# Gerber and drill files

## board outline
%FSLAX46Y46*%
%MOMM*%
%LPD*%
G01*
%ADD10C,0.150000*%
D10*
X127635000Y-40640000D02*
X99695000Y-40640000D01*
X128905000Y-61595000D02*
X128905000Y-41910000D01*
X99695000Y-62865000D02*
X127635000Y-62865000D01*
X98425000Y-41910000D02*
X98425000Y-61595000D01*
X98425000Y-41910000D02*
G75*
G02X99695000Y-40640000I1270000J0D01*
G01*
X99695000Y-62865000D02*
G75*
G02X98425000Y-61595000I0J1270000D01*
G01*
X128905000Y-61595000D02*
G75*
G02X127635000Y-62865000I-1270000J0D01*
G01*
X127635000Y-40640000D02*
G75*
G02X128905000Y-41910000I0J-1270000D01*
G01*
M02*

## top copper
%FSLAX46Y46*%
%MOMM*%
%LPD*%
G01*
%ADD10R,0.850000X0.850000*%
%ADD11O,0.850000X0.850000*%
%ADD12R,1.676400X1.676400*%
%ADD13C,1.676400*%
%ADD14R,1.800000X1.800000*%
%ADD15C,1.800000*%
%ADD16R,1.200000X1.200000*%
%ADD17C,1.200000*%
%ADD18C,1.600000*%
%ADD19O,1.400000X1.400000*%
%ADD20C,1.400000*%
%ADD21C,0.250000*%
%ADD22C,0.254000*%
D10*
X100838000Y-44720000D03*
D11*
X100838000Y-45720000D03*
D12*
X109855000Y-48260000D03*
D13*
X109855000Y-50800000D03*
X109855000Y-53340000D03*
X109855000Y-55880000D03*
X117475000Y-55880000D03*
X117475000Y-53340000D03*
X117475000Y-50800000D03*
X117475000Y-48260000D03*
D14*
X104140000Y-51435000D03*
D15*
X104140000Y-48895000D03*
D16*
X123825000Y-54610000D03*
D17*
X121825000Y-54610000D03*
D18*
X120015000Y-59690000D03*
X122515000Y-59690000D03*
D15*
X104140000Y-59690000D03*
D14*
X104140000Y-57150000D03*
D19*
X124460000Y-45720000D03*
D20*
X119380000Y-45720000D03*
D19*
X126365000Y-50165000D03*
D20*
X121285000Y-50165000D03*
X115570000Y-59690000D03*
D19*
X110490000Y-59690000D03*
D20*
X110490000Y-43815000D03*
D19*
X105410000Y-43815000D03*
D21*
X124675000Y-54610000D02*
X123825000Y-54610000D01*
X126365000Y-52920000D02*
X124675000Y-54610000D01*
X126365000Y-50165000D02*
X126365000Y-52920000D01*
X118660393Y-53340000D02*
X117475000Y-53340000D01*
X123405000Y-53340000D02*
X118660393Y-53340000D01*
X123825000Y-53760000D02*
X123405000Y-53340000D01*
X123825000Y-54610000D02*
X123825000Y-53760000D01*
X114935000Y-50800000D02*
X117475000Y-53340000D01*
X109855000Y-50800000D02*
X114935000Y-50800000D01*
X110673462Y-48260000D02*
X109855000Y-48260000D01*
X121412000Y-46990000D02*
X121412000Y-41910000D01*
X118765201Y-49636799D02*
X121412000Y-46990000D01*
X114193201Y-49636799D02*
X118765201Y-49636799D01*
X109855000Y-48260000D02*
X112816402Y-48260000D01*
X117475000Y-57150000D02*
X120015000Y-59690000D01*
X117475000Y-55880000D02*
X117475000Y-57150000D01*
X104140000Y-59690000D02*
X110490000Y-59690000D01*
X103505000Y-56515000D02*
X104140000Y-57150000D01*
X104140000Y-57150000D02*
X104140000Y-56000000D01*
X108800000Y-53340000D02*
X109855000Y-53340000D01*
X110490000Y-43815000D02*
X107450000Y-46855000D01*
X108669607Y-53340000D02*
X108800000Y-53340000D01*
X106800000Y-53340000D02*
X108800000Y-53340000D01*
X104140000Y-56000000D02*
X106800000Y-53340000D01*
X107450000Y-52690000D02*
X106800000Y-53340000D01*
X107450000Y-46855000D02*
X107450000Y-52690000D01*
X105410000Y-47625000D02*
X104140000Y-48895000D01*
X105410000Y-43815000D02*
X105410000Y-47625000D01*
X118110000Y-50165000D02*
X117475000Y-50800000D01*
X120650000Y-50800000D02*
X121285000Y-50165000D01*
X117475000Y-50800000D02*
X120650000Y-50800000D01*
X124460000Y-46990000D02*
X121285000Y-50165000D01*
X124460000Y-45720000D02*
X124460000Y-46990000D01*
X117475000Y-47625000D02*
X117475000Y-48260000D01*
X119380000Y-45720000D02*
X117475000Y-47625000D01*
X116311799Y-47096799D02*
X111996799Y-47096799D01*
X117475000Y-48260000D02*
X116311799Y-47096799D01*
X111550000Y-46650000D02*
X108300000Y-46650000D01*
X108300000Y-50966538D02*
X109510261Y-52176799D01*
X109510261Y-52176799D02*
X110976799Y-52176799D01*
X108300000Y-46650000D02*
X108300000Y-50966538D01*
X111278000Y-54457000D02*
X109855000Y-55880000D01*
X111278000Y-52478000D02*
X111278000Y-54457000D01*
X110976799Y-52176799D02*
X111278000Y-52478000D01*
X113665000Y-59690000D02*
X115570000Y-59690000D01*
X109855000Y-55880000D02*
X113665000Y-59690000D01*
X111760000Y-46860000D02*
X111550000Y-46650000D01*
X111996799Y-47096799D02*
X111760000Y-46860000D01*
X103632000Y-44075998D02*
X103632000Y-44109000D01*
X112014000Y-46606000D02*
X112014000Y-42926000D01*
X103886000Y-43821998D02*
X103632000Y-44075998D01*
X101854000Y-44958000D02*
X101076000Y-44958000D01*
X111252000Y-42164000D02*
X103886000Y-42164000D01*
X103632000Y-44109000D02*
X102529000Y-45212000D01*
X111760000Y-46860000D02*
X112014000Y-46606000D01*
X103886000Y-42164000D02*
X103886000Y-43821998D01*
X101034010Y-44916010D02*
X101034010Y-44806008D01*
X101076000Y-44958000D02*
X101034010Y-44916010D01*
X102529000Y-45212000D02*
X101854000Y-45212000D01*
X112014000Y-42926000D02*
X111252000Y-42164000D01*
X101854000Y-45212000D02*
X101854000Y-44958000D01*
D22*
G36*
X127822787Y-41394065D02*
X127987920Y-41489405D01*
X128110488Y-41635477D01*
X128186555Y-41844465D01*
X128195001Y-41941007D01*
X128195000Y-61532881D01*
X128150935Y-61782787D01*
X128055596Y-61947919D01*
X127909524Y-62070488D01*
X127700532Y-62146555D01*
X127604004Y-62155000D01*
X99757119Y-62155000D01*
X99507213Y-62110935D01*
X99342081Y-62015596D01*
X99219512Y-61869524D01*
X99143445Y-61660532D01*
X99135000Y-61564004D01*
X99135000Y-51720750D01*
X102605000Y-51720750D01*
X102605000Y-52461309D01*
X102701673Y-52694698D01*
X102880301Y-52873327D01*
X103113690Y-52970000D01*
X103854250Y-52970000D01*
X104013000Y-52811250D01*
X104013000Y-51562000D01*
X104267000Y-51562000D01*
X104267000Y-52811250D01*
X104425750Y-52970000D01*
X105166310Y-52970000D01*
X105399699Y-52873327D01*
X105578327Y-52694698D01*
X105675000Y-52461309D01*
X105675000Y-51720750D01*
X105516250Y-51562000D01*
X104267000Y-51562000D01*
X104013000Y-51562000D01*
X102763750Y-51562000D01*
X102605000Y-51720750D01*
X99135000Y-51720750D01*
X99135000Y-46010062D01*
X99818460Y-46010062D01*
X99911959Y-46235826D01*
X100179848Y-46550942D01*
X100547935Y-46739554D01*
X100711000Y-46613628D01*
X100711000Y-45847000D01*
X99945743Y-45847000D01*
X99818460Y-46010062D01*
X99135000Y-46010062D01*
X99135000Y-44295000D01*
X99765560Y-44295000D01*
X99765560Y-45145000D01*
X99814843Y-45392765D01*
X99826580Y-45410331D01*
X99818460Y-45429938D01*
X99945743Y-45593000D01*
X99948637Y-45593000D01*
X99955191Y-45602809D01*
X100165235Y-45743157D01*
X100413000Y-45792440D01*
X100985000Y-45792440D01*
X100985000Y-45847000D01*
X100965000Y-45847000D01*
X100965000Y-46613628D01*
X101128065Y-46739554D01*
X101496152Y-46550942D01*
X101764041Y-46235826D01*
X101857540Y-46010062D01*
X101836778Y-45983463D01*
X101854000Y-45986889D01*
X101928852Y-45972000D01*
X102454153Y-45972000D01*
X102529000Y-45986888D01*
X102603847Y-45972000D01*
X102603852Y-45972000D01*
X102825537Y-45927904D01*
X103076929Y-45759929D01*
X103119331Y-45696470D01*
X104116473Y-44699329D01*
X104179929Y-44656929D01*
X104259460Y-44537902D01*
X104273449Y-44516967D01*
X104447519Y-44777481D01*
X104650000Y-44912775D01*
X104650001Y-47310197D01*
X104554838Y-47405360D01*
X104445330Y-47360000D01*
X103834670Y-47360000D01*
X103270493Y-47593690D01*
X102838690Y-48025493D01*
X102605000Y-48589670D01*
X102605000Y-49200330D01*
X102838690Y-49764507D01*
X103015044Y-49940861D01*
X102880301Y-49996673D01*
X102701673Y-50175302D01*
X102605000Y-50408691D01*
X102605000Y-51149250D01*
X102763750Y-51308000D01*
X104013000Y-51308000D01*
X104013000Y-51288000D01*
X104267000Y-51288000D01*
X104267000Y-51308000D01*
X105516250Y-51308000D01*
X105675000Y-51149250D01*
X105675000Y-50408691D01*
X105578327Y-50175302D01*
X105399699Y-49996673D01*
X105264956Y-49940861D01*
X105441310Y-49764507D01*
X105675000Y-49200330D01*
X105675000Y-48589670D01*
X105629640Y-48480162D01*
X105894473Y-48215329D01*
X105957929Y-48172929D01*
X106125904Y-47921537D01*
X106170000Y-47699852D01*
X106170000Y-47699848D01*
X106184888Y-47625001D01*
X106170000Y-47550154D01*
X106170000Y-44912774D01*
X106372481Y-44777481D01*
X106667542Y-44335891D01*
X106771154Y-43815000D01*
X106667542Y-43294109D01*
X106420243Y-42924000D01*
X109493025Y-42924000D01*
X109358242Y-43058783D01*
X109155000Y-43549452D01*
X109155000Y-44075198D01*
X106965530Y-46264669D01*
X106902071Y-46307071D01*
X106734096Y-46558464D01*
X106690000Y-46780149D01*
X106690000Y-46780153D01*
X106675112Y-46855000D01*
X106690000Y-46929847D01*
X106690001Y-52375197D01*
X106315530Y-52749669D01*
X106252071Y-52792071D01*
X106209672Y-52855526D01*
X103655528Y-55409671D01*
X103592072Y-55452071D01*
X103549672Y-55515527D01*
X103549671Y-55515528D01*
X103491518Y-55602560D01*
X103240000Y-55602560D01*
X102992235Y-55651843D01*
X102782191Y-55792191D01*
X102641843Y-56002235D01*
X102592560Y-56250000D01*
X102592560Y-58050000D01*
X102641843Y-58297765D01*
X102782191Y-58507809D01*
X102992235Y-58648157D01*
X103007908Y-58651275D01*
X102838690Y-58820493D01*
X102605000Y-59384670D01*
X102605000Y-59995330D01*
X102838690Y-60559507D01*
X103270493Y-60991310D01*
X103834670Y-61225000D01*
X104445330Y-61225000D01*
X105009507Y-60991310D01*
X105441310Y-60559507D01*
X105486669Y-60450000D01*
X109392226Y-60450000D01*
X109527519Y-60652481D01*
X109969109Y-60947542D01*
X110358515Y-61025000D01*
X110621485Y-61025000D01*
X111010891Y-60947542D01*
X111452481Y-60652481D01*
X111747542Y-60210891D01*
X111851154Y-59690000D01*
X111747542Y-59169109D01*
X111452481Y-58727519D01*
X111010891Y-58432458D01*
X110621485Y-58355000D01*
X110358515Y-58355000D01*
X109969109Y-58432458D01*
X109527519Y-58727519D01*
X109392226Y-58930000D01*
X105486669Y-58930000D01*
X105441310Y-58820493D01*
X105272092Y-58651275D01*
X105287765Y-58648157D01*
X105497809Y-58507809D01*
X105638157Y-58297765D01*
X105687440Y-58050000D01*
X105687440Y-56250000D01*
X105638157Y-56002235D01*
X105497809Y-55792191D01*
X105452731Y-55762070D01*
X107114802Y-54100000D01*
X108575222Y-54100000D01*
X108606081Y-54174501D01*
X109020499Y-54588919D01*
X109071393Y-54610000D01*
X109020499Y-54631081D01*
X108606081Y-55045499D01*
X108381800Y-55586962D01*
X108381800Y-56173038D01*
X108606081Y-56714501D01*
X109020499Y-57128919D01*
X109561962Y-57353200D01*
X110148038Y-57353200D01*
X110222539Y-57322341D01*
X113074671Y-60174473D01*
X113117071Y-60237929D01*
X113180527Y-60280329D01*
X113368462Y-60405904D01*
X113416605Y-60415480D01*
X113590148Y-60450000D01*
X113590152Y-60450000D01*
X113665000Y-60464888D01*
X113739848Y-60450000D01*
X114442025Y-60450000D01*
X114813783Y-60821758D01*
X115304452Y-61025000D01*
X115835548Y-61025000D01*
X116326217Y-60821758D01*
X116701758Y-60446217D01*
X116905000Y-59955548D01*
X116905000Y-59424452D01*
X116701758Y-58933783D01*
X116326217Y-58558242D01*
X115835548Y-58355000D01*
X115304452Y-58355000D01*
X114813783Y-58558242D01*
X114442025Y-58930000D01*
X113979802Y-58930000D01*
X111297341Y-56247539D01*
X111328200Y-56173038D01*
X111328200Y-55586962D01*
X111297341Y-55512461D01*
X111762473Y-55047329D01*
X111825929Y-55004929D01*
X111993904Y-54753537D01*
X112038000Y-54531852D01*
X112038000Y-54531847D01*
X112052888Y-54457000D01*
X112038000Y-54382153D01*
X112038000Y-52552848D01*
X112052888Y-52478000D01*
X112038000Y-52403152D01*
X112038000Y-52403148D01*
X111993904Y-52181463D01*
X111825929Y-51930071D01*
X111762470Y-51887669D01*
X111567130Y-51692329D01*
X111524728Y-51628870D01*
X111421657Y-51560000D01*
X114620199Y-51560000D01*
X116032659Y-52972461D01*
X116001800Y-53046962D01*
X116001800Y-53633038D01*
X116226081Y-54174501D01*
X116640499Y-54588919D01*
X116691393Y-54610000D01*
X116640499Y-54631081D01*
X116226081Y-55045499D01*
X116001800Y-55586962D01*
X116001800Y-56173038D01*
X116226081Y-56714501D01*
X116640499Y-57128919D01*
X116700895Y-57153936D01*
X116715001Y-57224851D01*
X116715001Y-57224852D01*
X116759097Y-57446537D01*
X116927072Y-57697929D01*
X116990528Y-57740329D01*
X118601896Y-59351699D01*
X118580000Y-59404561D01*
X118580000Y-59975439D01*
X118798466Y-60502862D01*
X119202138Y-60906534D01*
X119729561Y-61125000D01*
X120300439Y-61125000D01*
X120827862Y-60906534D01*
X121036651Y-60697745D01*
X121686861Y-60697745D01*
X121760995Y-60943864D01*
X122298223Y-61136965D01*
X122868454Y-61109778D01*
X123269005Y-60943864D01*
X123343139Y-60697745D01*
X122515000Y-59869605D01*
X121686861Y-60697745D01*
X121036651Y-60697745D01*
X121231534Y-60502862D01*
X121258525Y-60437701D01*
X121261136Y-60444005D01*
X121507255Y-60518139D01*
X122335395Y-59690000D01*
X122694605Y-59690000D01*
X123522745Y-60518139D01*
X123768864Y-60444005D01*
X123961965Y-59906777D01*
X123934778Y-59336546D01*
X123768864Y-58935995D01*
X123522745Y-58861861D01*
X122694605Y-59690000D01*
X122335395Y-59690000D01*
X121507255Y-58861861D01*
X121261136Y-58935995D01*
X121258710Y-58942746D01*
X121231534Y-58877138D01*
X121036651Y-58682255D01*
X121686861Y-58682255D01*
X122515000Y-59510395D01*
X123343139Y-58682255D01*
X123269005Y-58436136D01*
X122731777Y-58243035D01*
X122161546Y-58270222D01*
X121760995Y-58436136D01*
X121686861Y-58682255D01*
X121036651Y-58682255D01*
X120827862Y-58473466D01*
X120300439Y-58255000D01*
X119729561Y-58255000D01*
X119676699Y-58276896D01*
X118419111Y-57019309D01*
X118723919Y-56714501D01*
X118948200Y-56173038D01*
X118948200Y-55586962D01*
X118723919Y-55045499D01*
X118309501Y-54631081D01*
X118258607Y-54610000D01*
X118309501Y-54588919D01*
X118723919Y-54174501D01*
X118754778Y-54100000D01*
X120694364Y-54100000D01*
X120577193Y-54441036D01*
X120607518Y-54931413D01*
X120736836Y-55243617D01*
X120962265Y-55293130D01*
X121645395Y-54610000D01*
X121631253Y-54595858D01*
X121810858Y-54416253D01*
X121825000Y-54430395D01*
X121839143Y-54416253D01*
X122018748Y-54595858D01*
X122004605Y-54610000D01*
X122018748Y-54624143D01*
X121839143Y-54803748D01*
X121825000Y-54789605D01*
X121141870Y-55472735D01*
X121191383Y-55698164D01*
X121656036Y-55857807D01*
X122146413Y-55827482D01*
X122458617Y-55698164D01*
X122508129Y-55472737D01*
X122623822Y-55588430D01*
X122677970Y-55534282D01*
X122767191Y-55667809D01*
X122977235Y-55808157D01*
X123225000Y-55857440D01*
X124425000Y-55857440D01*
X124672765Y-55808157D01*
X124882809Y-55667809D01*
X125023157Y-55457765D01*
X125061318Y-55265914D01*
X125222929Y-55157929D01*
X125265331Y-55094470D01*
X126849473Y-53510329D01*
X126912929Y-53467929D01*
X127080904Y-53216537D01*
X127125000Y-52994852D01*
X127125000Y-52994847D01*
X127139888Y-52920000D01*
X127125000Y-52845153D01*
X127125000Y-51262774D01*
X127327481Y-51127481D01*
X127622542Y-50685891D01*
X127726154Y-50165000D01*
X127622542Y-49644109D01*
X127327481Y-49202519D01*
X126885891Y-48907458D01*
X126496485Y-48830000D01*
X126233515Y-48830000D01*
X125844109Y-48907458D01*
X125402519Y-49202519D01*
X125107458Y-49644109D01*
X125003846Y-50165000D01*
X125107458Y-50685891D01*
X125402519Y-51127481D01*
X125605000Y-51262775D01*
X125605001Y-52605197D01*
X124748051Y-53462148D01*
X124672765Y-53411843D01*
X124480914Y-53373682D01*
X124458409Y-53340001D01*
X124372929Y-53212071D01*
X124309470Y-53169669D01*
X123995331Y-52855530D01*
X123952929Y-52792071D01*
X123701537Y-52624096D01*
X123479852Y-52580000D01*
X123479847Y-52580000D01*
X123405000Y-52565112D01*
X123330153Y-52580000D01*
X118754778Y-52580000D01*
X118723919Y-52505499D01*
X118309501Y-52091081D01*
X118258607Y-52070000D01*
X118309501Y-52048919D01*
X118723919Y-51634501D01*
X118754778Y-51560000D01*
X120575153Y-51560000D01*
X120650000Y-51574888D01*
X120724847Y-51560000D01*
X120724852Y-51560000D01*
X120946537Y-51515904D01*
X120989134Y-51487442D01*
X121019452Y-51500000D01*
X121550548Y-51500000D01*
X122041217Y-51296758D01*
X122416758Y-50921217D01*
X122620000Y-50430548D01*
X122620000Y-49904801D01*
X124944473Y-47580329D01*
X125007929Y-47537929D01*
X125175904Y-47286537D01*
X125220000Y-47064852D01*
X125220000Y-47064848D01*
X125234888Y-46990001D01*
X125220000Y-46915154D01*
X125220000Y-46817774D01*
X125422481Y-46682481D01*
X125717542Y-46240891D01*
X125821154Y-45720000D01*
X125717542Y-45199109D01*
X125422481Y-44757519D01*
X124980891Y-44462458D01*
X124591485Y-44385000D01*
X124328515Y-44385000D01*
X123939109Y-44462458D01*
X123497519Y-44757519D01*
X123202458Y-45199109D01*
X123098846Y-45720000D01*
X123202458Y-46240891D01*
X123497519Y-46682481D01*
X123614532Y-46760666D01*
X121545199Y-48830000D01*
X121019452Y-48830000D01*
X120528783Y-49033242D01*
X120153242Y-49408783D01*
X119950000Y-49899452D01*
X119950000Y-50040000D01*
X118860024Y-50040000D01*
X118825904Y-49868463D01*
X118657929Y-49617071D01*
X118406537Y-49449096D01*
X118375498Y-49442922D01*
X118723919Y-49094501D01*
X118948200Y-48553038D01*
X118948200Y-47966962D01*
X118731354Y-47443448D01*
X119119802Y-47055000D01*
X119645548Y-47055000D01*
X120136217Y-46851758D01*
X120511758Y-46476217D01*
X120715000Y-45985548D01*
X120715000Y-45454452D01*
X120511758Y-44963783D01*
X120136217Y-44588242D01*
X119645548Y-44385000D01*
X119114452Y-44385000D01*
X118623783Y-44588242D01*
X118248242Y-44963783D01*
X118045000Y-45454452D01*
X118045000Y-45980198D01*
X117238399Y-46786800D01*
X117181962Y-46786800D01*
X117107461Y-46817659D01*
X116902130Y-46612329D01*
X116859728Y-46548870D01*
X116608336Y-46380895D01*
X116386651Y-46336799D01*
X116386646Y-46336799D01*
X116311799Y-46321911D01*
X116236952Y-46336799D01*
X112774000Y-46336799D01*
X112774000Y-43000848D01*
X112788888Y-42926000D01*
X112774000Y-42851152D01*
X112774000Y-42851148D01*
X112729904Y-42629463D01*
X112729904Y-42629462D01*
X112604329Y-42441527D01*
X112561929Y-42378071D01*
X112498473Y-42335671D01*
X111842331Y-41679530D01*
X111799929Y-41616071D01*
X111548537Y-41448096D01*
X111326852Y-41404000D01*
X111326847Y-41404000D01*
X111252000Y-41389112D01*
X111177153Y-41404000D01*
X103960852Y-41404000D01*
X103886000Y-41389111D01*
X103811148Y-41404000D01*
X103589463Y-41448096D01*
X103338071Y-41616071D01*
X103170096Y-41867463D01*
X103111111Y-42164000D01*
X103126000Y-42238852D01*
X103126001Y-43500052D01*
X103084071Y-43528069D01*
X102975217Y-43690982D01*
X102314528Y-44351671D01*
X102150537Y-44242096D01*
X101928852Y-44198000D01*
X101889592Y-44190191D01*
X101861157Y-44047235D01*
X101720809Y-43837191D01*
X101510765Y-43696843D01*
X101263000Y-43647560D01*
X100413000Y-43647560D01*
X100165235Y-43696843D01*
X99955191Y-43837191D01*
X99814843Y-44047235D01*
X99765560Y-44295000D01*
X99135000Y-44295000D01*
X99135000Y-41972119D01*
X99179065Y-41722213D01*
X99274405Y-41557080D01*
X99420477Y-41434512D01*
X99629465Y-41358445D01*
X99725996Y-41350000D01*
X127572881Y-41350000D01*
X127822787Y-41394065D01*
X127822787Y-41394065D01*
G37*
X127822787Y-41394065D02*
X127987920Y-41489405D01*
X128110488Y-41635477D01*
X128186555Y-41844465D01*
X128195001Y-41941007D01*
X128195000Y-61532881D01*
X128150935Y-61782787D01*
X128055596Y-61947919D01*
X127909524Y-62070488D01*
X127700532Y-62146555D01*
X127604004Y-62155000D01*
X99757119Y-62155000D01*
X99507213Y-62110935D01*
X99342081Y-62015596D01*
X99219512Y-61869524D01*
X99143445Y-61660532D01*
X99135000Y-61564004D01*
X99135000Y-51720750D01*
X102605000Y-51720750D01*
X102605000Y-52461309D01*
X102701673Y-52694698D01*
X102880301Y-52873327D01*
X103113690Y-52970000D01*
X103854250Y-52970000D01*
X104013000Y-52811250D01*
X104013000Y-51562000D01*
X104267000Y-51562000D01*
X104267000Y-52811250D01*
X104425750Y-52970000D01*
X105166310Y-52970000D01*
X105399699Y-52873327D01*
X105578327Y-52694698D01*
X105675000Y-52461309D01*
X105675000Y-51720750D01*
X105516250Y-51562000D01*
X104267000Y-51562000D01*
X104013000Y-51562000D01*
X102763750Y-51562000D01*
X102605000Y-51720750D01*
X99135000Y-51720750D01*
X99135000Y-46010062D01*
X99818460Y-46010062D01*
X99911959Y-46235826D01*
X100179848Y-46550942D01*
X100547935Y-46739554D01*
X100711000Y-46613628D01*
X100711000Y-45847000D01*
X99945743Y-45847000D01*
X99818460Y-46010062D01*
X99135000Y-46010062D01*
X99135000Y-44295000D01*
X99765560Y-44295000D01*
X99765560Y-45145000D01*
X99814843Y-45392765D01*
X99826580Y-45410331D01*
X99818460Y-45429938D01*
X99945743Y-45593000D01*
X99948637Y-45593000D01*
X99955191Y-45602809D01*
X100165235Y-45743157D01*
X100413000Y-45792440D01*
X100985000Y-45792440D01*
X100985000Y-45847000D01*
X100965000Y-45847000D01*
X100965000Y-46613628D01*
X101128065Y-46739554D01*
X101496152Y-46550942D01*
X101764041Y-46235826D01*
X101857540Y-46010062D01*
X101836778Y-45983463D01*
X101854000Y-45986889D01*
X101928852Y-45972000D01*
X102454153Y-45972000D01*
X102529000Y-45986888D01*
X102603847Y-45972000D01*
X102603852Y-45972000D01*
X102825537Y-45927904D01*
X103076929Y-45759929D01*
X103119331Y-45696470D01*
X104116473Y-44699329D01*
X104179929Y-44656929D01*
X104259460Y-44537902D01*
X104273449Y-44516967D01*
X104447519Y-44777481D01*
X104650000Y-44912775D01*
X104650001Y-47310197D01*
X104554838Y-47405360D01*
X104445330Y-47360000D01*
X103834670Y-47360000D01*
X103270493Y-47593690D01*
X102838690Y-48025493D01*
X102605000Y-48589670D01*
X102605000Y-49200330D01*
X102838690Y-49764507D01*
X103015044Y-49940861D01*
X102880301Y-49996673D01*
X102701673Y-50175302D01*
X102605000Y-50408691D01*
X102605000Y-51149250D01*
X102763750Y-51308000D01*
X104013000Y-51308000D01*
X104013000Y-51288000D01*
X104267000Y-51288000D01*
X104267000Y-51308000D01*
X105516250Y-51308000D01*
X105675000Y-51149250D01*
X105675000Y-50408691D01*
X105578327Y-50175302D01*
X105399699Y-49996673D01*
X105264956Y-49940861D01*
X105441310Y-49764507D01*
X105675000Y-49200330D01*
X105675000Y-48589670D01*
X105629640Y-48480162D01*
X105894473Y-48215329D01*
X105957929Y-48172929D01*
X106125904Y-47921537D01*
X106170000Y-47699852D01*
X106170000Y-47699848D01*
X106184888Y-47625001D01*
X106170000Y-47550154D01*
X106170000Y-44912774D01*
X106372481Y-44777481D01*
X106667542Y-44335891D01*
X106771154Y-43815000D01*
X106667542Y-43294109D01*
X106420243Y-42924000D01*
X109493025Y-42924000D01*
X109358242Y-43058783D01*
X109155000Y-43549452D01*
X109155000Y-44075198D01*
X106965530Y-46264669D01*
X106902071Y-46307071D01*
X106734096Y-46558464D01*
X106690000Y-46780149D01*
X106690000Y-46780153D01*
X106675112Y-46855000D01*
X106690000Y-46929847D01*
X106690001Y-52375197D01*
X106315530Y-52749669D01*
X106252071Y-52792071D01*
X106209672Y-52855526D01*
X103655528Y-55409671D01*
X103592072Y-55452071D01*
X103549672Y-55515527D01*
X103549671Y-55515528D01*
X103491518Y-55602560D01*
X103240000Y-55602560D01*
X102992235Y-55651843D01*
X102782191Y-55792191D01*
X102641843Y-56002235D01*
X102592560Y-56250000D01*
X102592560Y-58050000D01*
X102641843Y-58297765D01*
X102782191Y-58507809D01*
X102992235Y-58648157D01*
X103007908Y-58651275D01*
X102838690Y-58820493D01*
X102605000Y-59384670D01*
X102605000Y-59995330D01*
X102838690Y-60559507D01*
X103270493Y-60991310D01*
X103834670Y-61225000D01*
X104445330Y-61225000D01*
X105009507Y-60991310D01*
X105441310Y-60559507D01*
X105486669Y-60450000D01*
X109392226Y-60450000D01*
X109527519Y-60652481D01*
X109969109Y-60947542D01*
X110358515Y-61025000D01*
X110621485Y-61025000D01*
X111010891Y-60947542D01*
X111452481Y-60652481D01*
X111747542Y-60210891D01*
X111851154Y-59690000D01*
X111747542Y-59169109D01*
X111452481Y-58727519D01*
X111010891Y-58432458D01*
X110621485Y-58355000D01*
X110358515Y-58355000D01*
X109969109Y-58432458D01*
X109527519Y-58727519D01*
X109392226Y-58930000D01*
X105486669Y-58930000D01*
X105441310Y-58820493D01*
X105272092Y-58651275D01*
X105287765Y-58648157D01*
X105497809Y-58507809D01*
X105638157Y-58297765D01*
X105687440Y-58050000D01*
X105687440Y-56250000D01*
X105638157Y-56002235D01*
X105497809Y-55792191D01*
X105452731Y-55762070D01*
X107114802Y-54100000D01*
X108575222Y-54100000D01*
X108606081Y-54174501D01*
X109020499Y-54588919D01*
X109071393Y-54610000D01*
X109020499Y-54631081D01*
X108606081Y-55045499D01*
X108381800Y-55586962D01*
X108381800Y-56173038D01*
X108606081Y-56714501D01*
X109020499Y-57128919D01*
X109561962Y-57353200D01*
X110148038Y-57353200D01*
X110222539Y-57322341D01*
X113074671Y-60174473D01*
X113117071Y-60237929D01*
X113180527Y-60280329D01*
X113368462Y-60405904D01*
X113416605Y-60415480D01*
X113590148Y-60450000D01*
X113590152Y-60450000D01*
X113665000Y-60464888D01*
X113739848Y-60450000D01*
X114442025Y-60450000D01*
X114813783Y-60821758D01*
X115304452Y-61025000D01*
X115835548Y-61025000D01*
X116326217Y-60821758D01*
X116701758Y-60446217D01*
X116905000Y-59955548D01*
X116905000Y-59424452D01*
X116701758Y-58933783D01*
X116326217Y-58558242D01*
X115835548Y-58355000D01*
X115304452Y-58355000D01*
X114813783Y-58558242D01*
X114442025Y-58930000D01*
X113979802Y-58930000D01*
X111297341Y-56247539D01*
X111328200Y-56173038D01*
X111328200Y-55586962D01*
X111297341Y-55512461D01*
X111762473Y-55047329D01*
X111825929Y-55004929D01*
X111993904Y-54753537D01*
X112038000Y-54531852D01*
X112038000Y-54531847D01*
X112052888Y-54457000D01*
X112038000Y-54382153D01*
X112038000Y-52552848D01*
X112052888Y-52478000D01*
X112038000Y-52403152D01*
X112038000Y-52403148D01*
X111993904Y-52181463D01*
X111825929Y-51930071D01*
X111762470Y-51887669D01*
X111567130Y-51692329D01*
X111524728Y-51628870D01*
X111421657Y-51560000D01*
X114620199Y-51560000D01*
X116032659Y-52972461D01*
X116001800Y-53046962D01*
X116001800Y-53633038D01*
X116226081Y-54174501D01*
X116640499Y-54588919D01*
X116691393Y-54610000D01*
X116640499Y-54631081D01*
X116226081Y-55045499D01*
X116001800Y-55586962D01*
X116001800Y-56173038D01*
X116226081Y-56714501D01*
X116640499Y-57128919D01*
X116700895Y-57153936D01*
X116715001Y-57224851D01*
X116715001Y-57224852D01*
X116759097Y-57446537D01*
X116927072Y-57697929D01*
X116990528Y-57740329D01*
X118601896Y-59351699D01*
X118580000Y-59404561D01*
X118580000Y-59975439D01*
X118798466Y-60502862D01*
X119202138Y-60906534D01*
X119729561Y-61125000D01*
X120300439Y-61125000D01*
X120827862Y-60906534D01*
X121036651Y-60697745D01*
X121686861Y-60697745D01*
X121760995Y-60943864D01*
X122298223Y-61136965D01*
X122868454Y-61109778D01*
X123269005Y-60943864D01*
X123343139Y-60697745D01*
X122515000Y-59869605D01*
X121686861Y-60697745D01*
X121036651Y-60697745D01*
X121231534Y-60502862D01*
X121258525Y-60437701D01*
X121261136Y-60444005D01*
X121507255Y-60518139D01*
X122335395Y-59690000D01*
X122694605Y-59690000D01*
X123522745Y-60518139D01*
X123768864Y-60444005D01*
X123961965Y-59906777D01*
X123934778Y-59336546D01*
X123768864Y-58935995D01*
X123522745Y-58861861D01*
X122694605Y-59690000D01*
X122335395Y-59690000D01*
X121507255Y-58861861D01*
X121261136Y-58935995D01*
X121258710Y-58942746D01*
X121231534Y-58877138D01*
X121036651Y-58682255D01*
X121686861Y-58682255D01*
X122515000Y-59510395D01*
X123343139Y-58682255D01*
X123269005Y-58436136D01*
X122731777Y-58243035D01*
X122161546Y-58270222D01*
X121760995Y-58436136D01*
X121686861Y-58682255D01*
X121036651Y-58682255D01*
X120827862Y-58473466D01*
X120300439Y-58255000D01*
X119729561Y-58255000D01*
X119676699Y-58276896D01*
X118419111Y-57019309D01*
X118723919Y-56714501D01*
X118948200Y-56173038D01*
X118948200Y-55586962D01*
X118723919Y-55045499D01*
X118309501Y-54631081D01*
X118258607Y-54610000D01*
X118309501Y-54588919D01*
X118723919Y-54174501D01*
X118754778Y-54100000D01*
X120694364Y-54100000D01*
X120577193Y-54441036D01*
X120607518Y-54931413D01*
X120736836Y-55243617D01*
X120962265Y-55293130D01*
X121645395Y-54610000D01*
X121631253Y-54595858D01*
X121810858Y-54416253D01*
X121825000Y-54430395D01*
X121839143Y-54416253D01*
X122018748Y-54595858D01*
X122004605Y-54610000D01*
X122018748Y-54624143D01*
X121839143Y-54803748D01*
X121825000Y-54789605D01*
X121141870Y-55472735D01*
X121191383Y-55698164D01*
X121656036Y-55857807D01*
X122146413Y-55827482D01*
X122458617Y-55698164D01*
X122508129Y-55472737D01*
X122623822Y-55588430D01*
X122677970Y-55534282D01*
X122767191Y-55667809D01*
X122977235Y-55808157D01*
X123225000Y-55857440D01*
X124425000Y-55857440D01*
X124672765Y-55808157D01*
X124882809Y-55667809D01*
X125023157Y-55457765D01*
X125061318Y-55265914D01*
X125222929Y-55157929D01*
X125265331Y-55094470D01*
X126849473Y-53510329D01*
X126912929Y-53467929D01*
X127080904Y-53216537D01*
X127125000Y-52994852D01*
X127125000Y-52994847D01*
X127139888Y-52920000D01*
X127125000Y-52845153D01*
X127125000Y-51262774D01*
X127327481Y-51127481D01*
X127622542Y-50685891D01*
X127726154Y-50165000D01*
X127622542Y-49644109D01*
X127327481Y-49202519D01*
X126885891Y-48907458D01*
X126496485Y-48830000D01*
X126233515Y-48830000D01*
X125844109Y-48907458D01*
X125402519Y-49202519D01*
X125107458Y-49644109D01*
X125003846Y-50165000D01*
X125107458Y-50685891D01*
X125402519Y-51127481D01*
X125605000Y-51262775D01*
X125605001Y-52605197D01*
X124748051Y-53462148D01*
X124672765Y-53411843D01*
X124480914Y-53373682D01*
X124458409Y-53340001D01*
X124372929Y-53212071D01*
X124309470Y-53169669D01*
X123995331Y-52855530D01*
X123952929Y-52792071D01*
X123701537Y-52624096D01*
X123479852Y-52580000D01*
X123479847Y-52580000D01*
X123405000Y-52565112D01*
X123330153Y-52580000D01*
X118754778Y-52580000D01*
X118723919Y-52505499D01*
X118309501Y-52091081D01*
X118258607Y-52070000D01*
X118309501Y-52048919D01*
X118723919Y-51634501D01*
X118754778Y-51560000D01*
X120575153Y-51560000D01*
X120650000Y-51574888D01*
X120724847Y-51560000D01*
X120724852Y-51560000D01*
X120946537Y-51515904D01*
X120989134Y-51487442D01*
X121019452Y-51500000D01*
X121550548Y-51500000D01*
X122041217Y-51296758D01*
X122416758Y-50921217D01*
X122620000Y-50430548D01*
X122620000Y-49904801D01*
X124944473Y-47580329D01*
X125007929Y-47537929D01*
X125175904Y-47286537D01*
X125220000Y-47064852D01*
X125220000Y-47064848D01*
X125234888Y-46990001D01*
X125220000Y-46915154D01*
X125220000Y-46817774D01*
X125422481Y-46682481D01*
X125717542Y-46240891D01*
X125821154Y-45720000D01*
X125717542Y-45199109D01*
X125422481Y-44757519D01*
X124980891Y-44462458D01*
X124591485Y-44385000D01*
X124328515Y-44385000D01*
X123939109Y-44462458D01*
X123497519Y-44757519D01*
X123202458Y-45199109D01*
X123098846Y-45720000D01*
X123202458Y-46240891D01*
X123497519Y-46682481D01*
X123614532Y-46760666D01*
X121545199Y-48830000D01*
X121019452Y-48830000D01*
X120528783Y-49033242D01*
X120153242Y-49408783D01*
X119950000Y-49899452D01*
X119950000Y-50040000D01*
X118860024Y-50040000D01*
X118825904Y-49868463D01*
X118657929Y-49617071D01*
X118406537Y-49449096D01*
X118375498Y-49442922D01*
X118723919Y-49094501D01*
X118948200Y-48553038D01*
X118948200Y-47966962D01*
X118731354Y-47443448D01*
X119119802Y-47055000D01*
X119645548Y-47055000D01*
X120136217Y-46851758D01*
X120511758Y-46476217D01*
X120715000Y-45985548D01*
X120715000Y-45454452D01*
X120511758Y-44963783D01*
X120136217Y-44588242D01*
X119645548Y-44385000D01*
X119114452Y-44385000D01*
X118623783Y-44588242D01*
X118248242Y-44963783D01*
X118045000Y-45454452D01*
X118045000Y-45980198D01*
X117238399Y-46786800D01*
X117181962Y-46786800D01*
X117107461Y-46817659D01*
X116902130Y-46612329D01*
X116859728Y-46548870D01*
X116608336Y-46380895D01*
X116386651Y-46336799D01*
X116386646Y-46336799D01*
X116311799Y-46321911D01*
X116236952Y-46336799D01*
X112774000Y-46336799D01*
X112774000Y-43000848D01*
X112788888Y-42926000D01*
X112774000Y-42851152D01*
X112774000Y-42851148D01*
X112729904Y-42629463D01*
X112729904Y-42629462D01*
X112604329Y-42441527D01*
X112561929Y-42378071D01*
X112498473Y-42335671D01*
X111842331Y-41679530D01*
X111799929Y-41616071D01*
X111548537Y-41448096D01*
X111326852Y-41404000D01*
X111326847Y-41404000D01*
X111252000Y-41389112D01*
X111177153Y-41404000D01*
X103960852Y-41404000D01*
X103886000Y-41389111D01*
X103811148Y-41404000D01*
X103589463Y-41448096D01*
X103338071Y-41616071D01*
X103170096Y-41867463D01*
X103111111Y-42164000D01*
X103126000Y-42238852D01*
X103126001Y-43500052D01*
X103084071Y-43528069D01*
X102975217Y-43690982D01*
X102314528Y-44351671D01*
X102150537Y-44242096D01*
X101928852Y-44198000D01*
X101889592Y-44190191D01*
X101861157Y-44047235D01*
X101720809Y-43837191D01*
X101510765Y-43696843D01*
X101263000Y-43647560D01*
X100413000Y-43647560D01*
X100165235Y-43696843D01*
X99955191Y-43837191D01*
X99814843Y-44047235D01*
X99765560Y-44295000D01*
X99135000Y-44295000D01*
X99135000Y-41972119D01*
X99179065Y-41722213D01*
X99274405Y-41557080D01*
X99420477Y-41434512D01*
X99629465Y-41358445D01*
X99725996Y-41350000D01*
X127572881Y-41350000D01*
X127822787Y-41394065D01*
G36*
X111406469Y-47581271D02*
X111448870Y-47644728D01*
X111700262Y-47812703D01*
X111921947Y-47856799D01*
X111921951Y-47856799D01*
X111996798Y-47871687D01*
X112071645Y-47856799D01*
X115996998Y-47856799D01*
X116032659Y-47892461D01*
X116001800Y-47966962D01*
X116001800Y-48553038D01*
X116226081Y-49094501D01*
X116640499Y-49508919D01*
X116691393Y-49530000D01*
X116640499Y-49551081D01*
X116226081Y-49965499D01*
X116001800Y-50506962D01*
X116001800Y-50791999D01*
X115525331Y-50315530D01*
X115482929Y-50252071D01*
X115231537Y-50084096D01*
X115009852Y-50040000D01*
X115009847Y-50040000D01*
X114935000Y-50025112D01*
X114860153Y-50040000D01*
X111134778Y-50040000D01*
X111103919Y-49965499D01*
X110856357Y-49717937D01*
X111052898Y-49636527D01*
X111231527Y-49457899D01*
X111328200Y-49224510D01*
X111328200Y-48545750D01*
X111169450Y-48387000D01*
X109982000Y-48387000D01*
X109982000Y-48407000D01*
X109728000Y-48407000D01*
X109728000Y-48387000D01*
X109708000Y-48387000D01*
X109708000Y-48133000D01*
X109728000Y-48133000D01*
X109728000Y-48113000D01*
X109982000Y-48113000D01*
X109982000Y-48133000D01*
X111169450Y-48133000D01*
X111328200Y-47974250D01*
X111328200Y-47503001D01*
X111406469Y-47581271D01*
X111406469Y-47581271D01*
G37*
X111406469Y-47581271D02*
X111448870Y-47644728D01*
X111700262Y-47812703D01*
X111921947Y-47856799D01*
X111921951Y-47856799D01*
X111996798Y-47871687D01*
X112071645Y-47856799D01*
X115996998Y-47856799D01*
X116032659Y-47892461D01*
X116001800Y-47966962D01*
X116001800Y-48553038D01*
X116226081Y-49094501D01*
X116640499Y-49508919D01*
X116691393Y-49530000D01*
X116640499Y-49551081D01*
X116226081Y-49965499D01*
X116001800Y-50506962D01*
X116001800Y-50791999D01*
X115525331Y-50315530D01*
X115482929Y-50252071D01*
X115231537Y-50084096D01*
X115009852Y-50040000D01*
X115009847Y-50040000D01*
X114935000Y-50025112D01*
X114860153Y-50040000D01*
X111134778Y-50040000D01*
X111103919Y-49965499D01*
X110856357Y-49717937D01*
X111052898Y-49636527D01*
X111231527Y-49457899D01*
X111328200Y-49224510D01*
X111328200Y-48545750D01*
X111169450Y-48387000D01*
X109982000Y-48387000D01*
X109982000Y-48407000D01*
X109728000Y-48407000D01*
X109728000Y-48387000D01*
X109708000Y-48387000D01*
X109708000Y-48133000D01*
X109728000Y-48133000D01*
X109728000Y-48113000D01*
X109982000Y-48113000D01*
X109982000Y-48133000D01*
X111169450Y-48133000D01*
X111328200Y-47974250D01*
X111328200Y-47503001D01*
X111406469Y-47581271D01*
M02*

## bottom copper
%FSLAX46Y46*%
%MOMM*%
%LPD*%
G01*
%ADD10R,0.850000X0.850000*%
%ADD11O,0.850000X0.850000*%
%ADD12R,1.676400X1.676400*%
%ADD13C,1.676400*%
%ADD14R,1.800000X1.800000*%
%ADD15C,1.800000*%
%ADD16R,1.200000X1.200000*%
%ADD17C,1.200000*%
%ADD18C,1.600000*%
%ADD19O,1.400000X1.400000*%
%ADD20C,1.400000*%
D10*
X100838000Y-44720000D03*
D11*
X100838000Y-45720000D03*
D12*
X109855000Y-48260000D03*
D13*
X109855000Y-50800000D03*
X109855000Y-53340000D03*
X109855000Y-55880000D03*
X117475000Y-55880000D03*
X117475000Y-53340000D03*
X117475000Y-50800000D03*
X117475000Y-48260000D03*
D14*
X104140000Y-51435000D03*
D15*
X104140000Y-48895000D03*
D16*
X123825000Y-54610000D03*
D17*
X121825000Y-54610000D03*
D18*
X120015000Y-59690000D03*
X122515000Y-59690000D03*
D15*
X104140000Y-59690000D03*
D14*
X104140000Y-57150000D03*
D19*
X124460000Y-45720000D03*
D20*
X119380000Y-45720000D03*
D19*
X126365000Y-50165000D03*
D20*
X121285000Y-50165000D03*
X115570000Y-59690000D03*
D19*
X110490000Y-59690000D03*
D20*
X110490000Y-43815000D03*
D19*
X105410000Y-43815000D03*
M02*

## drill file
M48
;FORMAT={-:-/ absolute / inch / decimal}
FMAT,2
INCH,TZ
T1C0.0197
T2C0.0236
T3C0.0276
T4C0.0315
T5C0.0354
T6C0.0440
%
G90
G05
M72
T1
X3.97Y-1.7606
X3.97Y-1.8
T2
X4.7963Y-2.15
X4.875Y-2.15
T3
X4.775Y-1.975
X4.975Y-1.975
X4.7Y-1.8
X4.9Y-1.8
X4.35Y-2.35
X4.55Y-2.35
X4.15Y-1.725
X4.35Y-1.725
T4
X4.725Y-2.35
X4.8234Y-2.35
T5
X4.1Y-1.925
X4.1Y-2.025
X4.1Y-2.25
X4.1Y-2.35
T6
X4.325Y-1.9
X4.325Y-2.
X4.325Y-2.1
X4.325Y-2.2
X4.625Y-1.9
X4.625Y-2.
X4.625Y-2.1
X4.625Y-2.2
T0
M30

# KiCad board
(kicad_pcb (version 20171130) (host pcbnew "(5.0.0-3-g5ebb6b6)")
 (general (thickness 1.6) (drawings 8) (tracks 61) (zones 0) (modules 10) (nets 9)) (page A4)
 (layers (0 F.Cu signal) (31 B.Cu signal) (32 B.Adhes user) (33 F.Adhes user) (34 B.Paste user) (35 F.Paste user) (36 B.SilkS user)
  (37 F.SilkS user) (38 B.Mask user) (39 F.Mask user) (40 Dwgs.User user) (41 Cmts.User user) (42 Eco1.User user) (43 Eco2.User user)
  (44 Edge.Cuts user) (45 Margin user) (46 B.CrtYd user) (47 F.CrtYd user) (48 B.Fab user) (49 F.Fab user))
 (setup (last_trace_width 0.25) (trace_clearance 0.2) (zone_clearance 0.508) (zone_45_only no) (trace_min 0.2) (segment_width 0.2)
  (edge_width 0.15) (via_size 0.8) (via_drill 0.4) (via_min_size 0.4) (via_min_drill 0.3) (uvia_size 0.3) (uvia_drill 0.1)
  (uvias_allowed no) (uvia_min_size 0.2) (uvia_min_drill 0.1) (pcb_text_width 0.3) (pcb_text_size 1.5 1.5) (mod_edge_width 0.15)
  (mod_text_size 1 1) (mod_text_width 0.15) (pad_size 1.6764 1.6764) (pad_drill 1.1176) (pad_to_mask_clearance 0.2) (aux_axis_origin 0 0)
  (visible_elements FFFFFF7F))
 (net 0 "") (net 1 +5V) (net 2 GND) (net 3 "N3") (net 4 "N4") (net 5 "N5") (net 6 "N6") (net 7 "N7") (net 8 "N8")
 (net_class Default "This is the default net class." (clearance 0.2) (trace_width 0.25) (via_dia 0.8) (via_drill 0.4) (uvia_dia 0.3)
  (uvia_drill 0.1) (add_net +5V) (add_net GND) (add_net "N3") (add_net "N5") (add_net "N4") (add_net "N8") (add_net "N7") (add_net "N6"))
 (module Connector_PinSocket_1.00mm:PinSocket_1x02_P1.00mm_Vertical (layer F.Cu) (at 100.838 44.72)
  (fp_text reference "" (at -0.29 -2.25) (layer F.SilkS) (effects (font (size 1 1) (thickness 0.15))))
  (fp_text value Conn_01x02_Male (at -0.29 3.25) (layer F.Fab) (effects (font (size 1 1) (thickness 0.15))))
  (pad 1 thru_hole rect (at 0 0) (size 0.85 0.85) (drill 0.5) (layers *.Cu *.Mask) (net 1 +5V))
  (pad 2 thru_hole oval (at 0 1) (size 0.85 0.85) (drill 0.5) (layers *.Cu *.Mask) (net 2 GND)))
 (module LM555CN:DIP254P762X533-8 (layer F.Cu) (at 117.475 55.88)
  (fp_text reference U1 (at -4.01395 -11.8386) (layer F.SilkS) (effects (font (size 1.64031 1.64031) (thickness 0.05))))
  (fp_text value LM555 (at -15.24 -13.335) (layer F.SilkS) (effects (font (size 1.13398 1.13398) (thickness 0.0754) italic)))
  (pad 1 thru_hole rect (at -7.62 -7.62) (size 1.6764 1.6764) (drill 1.1176) (layers *.Cu *.Mask) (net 2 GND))
  (pad 2 thru_hole circle (at -7.62 -5.08) (size 1.6764 1.6764) (drill 1.1176) (layers *.Cu *.Mask) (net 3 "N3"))
  (pad 3 thru_hole circle (at -7.62 -2.54) (size 1.6764 1.6764) (drill 1.1176) (layers *.Cu *.Mask) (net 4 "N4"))
  (pad 4 thru_hole circle (at -7.62 0) (size 1.6764 1.6764) (drill 1.1176) (layers *.Cu *.Mask) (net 1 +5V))
  (pad 5 thru_hole circle (at 0 0) (size 1.6764 1.6764) (drill 1.1176) (layers *.Cu *.Mask) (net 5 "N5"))
  (pad 6 thru_hole circle (at 0 -2.54) (size 1.6764 1.6764) (drill 1.1176) (layers *.Cu *.Mask) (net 3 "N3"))
  (pad 7 thru_hole circle (at 0 -5.08) (size 1.6764 1.6764) (drill 1.1176) (layers *.Cu *.Mask) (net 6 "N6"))
  (pad 8 thru_hole circle (at 0 -7.62) (size 1.6764 1.6764) (drill 1.1176) (layers *.Cu *.Mask) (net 1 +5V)))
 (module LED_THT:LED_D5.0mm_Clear (layer F.Cu) (at 104.14 51.435 90)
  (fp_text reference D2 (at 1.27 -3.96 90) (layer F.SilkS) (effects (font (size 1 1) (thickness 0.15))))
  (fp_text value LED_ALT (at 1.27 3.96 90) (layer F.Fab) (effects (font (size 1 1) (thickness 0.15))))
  (pad 1 thru_hole rect (at 0 0 90) (size 1.8 1.8) (drill 0.9) (layers *.Cu *.Mask) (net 2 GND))
  (pad 2 thru_hole circle (at 2.54 0 90) (size 1.8 1.8) (drill 0.9) (layers *.Cu *.Mask) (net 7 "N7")))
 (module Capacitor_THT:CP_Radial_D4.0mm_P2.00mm (layer F.Cu) (at 123.825 54.61 180)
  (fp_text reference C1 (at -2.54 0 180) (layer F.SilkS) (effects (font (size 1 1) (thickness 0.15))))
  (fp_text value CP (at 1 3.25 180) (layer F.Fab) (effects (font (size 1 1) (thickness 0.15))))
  (pad 1 thru_hole rect (at 0 0 180) (size 1.2 1.2) (drill 0.6) (layers *.Cu *.Mask) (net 3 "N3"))
  (pad 2 thru_hole circle (at 2 0 180) (size 1.2 1.2) (drill 0.6) (layers *.Cu *.Mask) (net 2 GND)))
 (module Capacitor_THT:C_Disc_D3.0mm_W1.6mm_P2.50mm (layer F.Cu) (at 120.015 59.69)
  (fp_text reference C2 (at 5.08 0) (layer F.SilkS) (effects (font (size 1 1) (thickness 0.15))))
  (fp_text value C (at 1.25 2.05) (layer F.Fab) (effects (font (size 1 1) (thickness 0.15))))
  (pad 1 thru_hole circle (at 0 0) (size 1.6 1.6) (drill 0.8) (layers *.Cu *.Mask) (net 5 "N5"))
  (pad 2 thru_hole circle (at 2.5 0) (size 1.6 1.6) (drill 0.8) (layers *.Cu *.Mask) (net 2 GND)))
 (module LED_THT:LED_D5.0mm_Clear (layer F.Cu) (at 104.14 57.15 270)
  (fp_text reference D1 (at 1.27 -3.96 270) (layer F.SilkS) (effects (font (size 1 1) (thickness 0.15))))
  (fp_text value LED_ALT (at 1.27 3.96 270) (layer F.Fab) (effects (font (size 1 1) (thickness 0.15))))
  (pad 2 thru_hole circle (at 2.54 0 270) (size 1.8 1.8) (drill 0.9) (layers *.Cu *.Mask) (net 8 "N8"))
  (pad 1 thru_hole rect (at 0 0 270) (size 1.8 1.8) (drill 0.9) (layers *.Cu *.Mask) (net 4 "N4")))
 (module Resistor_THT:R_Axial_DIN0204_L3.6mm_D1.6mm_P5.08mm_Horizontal (layer F.Cu) (at 119.38 45.72)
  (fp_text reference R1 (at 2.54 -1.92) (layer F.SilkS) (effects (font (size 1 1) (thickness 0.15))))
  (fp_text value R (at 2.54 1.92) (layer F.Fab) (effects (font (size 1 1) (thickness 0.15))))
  (pad 2 thru_hole oval (at 5.08 0) (size 1.4 1.4) (drill 0.7) (layers *.Cu *.Mask) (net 6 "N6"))
  (pad 1 thru_hole circle (at 0 0) (size 1.4 1.4) (drill 0.7) (layers *.Cu *.Mask) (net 1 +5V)))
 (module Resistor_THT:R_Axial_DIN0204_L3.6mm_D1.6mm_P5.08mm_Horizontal (layer F.Cu) (at 121.285 50.165)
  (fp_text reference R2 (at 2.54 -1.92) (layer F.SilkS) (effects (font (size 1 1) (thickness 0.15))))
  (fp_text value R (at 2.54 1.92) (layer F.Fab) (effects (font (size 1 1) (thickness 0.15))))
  (pad 2 thru_hole oval (at 5.08 0) (size 1.4 1.4) (drill 0.7) (layers *.Cu *.Mask) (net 3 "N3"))
  (pad 1 thru_hole circle (at 0 0) (size 1.4 1.4) (drill 0.7) (layers *.Cu *.Mask) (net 6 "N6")))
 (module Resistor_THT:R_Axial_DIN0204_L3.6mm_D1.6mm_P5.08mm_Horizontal (layer F.Cu) (at 115.57 59.69 180)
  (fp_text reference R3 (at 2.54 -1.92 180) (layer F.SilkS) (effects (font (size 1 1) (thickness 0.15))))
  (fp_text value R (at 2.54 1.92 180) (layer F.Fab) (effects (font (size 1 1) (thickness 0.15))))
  (pad 1 thru_hole circle (at 0 0 180) (size 1.4 1.4) (drill 0.7) (layers *.Cu *.Mask) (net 1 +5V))
  (pad 2 thru_hole oval (at 5.08 0 180) (size 1.4 1.4) (drill 0.7) (layers *.Cu *.Mask) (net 8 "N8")))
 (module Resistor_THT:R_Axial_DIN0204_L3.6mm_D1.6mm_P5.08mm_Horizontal (layer F.Cu) (at 110.49 43.815 180)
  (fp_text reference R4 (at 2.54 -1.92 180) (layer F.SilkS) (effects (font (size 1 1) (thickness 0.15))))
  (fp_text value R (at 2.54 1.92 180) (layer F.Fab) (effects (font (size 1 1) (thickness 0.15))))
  (pad 1 thru_hole circle (at 0 0 180) (size 1.4 1.4) (drill 0.7) (layers *.Cu *.Mask) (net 4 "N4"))
  (pad 2 thru_hole oval (at 5.08 0 180) (size 1.4 1.4) (drill 0.7) (layers *.Cu *.Mask) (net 7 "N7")))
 (gr_line (start 127.635 40.64) (end 99.695 40.64) (layer Edge.Cuts) (width 0.15))
 (gr_line (start 128.905 61.595) (end 128.905 41.91) (layer Edge.Cuts) (width 0.15))
 (gr_line (start 99.695 62.865) (end 127.635 62.865) (layer Edge.Cuts) (width 0.15))
 (gr_line (start 98.425 41.91) (end 98.425 61.595) (layer Edge.Cuts) (width 0.15))
 (gr_arc (start 99.695 41.91) (end 99.695 40.64) (angle -90) (layer Edge.Cuts) (width 0.15))
 (gr_arc (start 99.695 61.595) (end 98.425 61.595) (angle -90) (layer Edge.Cuts) (width 0.15))
 (gr_arc (start 127.635 61.595) (end 127.635 62.865) (angle -90) (layer Edge.Cuts) (width 0.15))
 (gr_arc (start 127.635 41.91) (end 128.905 41.91) (angle -90) (layer Edge.Cuts) (width 0.15))
 (segment (start 124.675 54.61) (end 123.825 54.61) (width 0.25) (layer F.Cu) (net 3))
 (segment (start 126.365 52.92) (end 124.675 54.61) (width 0.25) (layer F.Cu) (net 3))
 (segment (start 126.365 50.165) (end 126.365 52.92) (width 0.25) (layer F.Cu) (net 3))
 (segment (start 118.660393 53.34) (end 117.475 53.34) (width 0.25) (layer F.Cu) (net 3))
 (segment (start 123.405 53.34) (end 118.660393 53.34) (width 0.25) (layer F.Cu) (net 3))
 (segment (start 123.825 53.76) (end 123.405 53.34) (width 0.25) (layer F.Cu) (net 3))
 (segment (start 123.825 54.61) (end 123.825 53.76) (width 0.25) (layer F.Cu) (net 3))
 (segment (start 114.935 50.8) (end 117.475 53.34) (width 0.25) (layer F.Cu) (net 3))
 (segment (start 109.855 50.8) (end 114.935 50.8) (width 0.25) (layer F.Cu) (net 3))
 (segment (start 110.673462 48.26) (end 109.855 48.26) (width 0.25) (layer F.Cu) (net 2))
 (segment (start 121.412 46.99) (end 121.412 41.91) (width 0.25) (layer F.Cu) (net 2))
 (segment (start 118.765201 49.636799) (end 121.412 46.99) (width 0.25) (layer F.Cu) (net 2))
 (segment (start 114.193201 49.636799) (end 118.765201 49.636799) (width 0.25) (layer F.Cu) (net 2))
 (segment (start 109.855 48.26) (end 112.816402 48.26) (width 0.25) (layer F.Cu) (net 2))
 (segment (start 117.475 57.15) (end 120.015 59.69) (width 0.25) (layer F.Cu) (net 5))
 (segment (start 117.475 55.88) (end 117.475 57.15) (width 0.25) (layer F.Cu) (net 5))
 (segment (start 104.14 59.69) (end 110.49 59.69) (width 0.25) (layer F.Cu) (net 8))
 (segment (start 103.505 56.515) (end 104.14 57.15) (width 0.25) (layer F.Cu) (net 4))
 (segment (start 104.14 57.15) (end 104.14 56) (width 0.25) (layer F.Cu) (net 4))
 (segment (start 108.8 53.34) (end 109.855 53.34) (width 0.25) (layer F.Cu) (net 4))
 (segment (start 110.49 43.815) (end 107.45 46.855) (width 0.25) (layer F.Cu) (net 4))
 (segment (start 108.669607 53.34) (end 108.8 53.34) (width 0.25) (layer F.Cu) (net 4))
 (segment (start 106.8 53.34) (end 108.8 53.34) (width 0.25) (layer F.Cu) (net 4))
 (segment (start 104.14 56) (end 106.8 53.34) (width 0.25) (layer F.Cu) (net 4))
 (segment (start 107.45 52.69) (end 106.8 53.34) (width 0.25) (layer F.Cu) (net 4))
 (segment (start 107.45 46.855) (end 107.45 52.69) (width 0.25) (layer F.Cu) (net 4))
 (segment (start 105.41 47.625) (end 104.14 48.895) (width 0.25) (layer F.Cu) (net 7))
 (segment (start 105.41 43.815) (end 105.41 47.625) (width 0.25) (layer F.Cu) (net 7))
 (segment (start 118.11 50.165) (end 117.475 50.8) (width 0.25) (layer F.Cu) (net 6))
 (segment (start 120.65 50.8) (end 121.285 50.165) (width 0.25) (layer F.Cu) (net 6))
 (segment (start 117.475 50.8) (end 120.65 50.8) (width 0.25) (layer F.Cu) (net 6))
 (segment (start 124.46 46.99) (end 121.285 50.165) (width 0.25) (layer F.Cu) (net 6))
 (segment (start 124.46 45.72) (end 124.46 46.99) (width 0.25) (layer F.Cu) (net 6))
 (segment (start 117.475 47.625) (end 117.475 48.26) (width 0.25) (layer F.Cu) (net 1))
 (segment (start 119.38 45.72) (end 117.475 47.625) (width 0.25) (layer F.Cu) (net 1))
 (segment (start 116.311799 47.096799) (end 111.996799 47.096799) (width 0.25) (layer F.Cu) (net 1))
 (segment (start 117.475 48.26) (end 116.311799 47.096799) (width 0.25) (layer F.Cu) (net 1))
 (segment (start 111.55 46.65) (end 108.3 46.65) (width 0.25) (layer F.Cu) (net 1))
 (segment (start 108.3 50.966538) (end 109.510261 52.176799) (width 0.25) (layer F.Cu) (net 1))
 (segment (start 109.510261 52.176799) (end 110.976799 52.176799) (width 0.25) (layer F.Cu) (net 1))
 (segment (start 108.3 46.65) (end 108.3 50.966538) (width 0.25) (layer F.Cu) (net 1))
 (segment (start 111.278 54.457) (end 109.855 55.88) (width 0.25) (layer F.Cu) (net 1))
 (segment (start 111.278 52.478) (end 111.278 54.457) (width 0.25) (layer F.Cu) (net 1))
 (segment (start 110.976799 52.176799) (end 111.278 52.478) (width 0.25) (layer F.Cu) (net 1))
 (segment (start 113.665 59.69) (end 115.57 59.69) (width 0.25) (layer F.Cu) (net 1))
 (segment (start 109.855 55.88) (end 113.665 59.69) (width 0.25) (layer F.Cu) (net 1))
 (segment (start 111.76 46.86) (end 111.55 46.65) (width 0.25) (layer F.Cu) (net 1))
 (segment (start 111.996799 47.096799) (end 111.76 46.86) (width 0.25) (layer F.Cu) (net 1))
 (segment (start 103.632 44.075998) (end 103.632 44.109) (width 0.25) (layer F.Cu) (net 1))
 (segment (start 112.014 46.606) (end 112.014 42.926) (width 0.25) (layer F.Cu) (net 1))
 (segment (start 103.886 43.821998) (end 103.632 44.075998) (width 0.25) (layer F.Cu) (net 1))
 (segment (start 101.854 44.958) (end 101.076 44.958) (width 0.25) (layer F.Cu) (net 1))
 (segment (start 111.252 42.164) (end 103.886 42.164) (width 0.25) (layer F.Cu) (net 1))
 (segment (start 103.632 44.109) (end 102.529 45.212) (width 0.25) (layer F.Cu) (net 1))
 (segment (start 111.76 46.86) (end 112.014 46.606) (width 0.25) (layer F.Cu) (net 1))
 (segment (start 103.886 42.164) (end 103.886 43.821998) (width 0.25) (layer F.Cu) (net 1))
 (segment (start 101.03401 44.91601) (end 101.03401 44.806008) (width 0.25) (layer F.Cu) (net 1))
 (segment (start 101.076 44.958) (end 101.03401 44.91601) (width 0.25) (layer F.Cu) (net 1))
 (segment (start 102.529 45.212) (end 101.854 45.212) (width 0.25) (layer F.Cu) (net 1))
 (segment (start 112.014 42.926) (end 111.252 42.164) (width 0.25) (layer F.Cu) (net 1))
 (segment (start 101.854 45.212) (end 101.854 44.958) (width 0.25) (layer F.Cu) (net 1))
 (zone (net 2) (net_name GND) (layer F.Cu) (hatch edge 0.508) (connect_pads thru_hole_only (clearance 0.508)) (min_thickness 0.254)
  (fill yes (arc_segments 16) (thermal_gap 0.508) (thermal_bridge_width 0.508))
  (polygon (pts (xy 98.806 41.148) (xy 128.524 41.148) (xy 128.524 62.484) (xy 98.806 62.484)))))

